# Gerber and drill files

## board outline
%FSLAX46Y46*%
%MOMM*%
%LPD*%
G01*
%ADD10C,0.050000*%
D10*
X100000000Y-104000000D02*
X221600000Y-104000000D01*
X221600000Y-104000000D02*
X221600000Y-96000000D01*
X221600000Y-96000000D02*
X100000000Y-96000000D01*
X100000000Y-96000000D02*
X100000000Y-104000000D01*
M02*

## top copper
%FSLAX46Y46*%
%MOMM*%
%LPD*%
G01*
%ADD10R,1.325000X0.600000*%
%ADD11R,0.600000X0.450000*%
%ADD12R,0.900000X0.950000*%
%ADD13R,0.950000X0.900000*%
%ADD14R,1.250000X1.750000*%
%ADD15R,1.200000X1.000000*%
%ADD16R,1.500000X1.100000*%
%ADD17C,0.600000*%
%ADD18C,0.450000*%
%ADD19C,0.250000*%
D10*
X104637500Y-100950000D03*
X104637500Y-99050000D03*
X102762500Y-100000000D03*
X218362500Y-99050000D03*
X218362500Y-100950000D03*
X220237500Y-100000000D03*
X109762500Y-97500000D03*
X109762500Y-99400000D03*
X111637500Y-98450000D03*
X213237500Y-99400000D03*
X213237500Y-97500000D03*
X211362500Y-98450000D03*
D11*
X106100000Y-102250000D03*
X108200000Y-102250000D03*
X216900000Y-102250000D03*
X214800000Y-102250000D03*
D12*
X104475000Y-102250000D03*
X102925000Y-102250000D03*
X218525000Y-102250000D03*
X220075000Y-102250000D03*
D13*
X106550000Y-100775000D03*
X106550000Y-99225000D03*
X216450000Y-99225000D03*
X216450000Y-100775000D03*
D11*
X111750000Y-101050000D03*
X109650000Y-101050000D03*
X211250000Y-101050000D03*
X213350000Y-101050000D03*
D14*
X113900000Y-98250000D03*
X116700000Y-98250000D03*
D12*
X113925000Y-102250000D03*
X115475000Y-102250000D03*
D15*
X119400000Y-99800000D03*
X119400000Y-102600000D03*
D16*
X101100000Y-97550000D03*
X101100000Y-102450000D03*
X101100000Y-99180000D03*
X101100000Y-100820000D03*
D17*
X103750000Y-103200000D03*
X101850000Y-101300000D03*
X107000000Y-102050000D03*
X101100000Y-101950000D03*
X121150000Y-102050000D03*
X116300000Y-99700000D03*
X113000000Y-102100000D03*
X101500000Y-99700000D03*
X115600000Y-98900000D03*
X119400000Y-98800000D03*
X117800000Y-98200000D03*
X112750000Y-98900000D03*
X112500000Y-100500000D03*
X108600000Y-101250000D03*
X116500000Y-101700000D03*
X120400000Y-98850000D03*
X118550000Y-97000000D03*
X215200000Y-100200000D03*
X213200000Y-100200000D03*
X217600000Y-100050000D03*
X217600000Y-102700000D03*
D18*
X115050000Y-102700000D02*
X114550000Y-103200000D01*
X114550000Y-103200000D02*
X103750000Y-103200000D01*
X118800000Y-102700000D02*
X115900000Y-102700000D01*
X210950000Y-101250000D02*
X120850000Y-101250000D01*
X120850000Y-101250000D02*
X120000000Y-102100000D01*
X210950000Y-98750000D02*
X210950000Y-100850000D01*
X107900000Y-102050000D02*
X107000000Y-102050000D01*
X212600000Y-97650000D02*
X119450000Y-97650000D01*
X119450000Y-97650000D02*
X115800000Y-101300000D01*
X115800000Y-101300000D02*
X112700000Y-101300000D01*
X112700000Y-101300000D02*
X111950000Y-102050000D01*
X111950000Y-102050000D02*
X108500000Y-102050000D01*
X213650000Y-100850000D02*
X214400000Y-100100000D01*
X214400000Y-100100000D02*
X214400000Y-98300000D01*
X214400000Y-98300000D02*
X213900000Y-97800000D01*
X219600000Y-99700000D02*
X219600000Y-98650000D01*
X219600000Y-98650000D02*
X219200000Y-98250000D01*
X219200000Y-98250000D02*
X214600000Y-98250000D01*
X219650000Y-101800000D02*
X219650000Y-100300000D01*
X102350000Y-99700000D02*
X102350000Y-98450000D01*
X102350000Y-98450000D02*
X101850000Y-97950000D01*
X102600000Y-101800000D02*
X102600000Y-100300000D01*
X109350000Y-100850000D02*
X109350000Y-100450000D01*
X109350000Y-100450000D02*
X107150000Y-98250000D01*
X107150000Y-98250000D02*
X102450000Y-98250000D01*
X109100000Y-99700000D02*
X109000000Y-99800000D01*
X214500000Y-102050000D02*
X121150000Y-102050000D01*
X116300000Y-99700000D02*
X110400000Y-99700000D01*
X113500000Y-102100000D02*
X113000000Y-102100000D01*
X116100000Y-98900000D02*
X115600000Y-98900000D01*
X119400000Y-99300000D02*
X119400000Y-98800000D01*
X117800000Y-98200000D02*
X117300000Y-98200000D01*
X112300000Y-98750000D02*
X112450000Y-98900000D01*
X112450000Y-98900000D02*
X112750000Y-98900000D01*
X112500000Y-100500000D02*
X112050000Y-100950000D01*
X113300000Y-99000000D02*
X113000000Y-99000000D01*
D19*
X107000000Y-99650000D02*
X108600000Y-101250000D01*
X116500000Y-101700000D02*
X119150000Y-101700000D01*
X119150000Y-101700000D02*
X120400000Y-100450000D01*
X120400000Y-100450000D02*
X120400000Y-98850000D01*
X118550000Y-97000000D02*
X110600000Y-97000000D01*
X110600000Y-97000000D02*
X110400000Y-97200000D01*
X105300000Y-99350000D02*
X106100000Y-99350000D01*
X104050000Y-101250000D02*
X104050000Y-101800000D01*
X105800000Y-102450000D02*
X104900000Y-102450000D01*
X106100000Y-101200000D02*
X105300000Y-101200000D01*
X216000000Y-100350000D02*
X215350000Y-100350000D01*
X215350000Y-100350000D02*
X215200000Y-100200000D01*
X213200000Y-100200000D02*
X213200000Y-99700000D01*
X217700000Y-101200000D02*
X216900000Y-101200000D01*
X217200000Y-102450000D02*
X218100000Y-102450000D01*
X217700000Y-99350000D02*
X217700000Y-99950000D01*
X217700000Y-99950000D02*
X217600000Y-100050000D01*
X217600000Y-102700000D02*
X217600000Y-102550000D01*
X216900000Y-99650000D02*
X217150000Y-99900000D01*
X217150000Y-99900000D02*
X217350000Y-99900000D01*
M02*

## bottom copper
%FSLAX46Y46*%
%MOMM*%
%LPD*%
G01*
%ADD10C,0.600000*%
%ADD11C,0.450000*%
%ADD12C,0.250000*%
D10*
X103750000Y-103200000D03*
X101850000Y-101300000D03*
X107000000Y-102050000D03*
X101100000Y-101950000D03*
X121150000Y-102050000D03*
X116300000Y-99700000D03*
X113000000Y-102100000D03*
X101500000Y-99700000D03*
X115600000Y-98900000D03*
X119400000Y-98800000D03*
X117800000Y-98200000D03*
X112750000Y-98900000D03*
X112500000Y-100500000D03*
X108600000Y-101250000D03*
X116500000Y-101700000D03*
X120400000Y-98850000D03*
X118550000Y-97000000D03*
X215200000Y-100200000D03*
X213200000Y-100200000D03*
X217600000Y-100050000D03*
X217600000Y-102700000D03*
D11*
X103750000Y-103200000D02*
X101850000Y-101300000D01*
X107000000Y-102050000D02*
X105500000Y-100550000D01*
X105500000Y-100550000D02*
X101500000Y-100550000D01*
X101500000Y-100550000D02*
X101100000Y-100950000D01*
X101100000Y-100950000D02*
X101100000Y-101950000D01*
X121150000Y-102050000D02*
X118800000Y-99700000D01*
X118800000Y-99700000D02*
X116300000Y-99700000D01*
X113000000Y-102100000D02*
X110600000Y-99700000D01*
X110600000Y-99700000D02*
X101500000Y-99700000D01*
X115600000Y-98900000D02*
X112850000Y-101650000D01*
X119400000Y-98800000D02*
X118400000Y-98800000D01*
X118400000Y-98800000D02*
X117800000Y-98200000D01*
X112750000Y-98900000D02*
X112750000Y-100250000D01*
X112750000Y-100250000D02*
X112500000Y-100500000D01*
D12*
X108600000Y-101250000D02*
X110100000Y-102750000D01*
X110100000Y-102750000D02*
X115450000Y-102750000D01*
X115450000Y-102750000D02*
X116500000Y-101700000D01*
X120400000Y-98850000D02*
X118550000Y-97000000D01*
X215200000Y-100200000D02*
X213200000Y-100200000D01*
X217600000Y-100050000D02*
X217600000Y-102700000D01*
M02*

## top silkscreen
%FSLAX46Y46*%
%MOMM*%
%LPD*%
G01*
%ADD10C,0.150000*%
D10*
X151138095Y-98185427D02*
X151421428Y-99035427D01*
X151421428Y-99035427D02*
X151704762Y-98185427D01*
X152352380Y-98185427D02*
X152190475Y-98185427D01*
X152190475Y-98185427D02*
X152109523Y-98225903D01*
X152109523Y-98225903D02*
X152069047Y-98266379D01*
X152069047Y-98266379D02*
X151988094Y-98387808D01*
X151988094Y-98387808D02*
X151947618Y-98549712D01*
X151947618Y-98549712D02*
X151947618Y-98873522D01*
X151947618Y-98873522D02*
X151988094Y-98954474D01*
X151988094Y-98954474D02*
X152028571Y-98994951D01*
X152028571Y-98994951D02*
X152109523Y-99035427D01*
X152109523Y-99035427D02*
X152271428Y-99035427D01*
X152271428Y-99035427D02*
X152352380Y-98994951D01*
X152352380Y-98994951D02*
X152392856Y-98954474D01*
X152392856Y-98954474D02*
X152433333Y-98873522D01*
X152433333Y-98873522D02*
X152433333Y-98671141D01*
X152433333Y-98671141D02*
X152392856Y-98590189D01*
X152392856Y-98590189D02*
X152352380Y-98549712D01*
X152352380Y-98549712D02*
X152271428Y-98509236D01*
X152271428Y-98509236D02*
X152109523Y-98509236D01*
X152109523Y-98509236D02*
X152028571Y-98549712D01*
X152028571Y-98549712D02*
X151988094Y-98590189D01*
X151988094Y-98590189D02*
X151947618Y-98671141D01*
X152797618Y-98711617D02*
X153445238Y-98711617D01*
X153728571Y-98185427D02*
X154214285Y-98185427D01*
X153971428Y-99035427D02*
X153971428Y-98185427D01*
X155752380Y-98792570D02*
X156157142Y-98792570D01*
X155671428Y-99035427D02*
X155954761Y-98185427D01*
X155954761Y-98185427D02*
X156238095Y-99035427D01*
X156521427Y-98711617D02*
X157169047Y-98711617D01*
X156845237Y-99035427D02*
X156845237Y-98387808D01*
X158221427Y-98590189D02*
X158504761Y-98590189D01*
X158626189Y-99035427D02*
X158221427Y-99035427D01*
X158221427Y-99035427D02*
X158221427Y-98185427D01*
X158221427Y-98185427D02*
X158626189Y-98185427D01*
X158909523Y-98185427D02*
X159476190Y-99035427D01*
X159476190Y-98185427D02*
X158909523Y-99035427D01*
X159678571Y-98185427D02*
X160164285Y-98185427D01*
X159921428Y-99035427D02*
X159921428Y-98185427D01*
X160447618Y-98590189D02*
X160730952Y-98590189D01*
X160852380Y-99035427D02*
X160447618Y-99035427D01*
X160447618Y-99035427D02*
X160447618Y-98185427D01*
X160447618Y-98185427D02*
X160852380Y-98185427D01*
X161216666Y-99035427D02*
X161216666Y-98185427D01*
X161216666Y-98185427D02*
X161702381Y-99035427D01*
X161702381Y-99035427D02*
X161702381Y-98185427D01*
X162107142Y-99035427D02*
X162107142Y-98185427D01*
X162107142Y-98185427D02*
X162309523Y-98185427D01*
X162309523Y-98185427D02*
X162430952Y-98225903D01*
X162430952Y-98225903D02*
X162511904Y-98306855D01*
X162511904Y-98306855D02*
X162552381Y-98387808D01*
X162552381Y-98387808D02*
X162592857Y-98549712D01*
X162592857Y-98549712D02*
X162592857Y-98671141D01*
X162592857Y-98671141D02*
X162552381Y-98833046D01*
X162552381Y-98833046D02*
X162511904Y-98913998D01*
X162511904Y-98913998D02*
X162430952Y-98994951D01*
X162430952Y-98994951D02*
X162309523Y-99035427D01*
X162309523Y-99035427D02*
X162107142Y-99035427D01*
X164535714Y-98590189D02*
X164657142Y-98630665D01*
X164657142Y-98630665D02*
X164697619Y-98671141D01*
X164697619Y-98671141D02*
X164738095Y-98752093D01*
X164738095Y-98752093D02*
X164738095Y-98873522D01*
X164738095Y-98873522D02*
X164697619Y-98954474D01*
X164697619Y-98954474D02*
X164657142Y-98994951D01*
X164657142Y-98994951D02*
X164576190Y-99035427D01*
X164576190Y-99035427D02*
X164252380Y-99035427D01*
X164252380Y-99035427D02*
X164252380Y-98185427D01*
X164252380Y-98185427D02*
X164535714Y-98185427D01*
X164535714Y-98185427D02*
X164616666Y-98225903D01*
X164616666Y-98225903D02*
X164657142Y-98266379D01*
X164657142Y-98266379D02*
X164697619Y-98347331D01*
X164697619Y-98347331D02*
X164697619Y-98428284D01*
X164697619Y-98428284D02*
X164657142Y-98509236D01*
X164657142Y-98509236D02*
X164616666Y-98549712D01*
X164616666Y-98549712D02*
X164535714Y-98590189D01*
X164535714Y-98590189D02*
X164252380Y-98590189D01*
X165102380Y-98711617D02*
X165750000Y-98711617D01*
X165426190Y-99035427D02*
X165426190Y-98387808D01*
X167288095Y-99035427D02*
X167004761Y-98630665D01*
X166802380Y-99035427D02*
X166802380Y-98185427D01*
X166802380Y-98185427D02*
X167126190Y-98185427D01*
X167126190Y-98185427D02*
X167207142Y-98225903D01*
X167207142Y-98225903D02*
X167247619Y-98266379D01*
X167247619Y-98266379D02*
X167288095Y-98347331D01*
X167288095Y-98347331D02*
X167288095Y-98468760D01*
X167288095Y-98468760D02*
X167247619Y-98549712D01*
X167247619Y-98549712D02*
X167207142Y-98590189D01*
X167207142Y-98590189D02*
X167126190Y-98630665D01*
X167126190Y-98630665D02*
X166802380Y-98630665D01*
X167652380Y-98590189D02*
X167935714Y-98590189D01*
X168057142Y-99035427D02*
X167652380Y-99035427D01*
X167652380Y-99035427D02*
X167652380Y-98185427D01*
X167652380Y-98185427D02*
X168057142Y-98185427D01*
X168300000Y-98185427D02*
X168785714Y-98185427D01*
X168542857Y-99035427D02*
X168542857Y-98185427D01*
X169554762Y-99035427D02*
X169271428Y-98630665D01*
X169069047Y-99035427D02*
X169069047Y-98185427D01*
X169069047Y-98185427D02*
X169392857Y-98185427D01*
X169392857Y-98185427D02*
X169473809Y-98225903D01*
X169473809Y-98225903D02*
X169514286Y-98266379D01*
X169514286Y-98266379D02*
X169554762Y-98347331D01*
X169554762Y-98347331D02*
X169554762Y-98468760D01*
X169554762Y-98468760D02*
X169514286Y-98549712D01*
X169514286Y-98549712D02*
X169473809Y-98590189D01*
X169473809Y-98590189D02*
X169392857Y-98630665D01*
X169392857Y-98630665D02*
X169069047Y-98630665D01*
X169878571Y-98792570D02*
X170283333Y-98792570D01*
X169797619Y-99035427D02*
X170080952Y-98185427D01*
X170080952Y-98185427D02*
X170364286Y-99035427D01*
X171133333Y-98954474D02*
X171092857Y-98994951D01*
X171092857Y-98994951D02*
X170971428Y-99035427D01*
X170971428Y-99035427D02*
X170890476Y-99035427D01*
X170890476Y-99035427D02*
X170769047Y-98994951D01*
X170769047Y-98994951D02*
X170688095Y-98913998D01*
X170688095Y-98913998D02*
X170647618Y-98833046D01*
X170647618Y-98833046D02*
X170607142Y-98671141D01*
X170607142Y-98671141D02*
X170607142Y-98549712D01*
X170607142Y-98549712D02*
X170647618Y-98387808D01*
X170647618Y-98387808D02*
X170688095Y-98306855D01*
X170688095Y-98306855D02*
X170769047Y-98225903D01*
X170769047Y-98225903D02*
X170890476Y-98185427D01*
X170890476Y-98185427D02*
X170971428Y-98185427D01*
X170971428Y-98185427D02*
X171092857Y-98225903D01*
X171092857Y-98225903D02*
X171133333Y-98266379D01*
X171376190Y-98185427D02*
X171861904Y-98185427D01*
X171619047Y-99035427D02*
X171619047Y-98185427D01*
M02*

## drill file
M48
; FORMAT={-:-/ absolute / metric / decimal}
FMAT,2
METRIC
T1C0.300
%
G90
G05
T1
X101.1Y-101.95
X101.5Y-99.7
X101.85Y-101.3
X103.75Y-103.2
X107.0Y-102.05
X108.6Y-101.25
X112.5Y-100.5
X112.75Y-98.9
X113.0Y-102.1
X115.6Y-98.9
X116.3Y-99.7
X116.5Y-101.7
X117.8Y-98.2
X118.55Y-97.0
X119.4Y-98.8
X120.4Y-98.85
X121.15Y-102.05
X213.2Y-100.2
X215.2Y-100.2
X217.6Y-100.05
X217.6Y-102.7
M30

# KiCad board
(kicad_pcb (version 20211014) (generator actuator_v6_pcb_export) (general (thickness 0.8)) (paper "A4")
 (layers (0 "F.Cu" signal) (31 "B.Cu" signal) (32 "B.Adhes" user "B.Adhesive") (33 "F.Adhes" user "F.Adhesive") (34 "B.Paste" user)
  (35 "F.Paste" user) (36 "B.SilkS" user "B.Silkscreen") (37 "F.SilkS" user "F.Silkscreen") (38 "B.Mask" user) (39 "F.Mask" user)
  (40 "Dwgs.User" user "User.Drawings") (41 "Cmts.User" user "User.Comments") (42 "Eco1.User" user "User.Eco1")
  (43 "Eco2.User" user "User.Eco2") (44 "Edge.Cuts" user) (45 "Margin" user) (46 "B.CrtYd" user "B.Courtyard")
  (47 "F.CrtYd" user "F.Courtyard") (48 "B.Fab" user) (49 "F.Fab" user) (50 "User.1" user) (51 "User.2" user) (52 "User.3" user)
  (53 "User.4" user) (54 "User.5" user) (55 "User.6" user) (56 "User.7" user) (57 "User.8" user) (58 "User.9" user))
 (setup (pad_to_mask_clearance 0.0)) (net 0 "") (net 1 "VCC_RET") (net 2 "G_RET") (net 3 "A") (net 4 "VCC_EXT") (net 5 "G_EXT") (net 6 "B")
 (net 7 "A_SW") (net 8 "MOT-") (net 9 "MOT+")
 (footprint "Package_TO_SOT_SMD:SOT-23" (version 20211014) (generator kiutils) (layer "F.Cu") (at 103.7 100.0 180)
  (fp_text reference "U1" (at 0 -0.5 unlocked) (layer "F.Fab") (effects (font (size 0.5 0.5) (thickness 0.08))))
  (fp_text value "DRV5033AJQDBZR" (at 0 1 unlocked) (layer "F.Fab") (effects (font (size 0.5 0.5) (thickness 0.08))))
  (pad "1" smd rect (at -0.9375 -0.95 180) (size 1.325 0.6) (layers "F.Cu" "F.Mask" "F.Paste") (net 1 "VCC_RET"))
  (pad "2" smd rect (at -0.9375 0.95 180) (size 1.325 0.6) (layers "F.Cu" "F.Mask" "F.Paste") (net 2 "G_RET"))
  (pad "3" smd rect (at 0.9375 0.0 180) (size 1.325 0.6) (layers "F.Cu" "F.Mask" "F.Paste") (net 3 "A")))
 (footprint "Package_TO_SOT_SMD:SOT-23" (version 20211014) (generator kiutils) (layer "F.Cu") (at 219.3 100.0)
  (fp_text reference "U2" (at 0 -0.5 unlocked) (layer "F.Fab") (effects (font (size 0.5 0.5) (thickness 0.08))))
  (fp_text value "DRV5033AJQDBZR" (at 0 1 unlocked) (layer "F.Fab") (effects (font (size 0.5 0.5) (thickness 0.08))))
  (pad "1" smd rect (at -0.9375 -0.95) (size 1.325 0.6) (layers "F.Cu" "F.Mask" "F.Paste") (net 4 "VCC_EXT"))
  (pad "2" smd rect (at -0.9375 0.95) (size 1.325 0.6) (layers "F.Cu" "F.Mask" "F.Paste") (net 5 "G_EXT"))
  (pad "3" smd rect (at 0.9375 0.0) (size 1.325 0.6) (layers "F.Cu" "F.Mask" "F.Paste") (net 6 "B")))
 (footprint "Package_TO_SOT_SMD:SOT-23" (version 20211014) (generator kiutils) (layer "F.Cu") (at 110.7 98.45)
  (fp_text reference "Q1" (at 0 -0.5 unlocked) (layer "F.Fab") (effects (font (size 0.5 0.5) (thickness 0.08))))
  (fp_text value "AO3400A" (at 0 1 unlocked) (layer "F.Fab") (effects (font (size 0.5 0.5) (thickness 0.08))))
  (pad "1" smd rect (at -0.9375 -0.95) (size 1.325 0.6) (layers "F.Cu" "F.Mask" "F.Paste") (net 2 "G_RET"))
  (pad "2" smd rect (at -0.9375 0.95) (size 1.325 0.6) (layers "F.Cu" "F.Mask" "F.Paste") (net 3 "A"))
  (pad "3" smd rect (at 0.9375 0.0) (size 1.325 0.6) (layers "F.Cu" "F.Mask" "F.Paste") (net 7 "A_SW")))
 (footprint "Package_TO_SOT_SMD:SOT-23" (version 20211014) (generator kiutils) (layer "F.Cu") (at 212.3 98.45 180)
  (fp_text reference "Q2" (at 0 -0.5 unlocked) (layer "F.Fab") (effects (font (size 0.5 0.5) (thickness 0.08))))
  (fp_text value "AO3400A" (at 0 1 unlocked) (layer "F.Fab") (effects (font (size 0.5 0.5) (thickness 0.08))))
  (pad "1" smd rect (at -0.9375 -0.95 180) (size 1.325 0.6) (layers "F.Cu" "F.Mask" "F.Paste") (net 5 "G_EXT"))
  (pad "2" smd rect (at -0.9375 0.95 180) (size 1.325 0.6) (layers "F.Cu" "F.Mask" "F.Paste") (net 6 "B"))
  (pad "3" smd rect (at 0.9375 0.0 180) (size 1.325 0.6) (layers "F.Cu" "F.Mask" "F.Paste") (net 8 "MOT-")))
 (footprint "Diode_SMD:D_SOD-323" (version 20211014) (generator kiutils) (layer "F.Cu") (at 107.15 102.25)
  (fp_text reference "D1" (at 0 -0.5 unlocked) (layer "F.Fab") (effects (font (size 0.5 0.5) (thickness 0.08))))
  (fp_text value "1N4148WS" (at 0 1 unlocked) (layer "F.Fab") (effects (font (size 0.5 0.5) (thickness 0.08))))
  (pad "1" smd rect (at -1.05 0.0) (size 0.6 0.45) (layers "F.Cu" "F.Mask" "F.Paste") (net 1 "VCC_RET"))
  (pad "2" smd rect (at 1.05 0.0) (size 0.6 0.45) (layers "F.Cu" "F.Mask" "F.Paste") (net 6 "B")))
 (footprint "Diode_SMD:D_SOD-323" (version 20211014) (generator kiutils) (layer "F.Cu") (at 215.85 102.25 180)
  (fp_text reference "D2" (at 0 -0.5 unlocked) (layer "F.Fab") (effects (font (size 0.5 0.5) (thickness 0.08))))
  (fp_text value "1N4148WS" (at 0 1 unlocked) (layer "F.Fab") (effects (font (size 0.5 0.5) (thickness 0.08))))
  (pad "1" smd rect (at -1.05 0.0 180) (size 0.6 0.45) (layers "F.Cu" "F.Mask" "F.Paste") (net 4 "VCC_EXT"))
  (pad "2" smd rect (at 1.05 0.0 180) (size 0.6 0.45) (layers "F.Cu" "F.Mask" "F.Paste") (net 3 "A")))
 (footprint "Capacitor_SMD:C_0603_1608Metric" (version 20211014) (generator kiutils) (layer "F.Cu") (at 103.7 102.25 180)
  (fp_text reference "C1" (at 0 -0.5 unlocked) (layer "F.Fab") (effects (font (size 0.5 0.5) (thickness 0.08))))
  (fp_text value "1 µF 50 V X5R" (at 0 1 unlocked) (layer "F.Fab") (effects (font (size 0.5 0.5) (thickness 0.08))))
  (pad "1" smd rect (at -0.775 0.0 180) (size 0.9 0.95) (layers "F.Cu" "F.Mask" "F.Paste") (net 1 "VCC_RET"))
  (pad "2" smd rect (at 0.775 0.0 180) (size 0.9 0.95) (layers "F.Cu" "F.Mask" "F.Paste") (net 3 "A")))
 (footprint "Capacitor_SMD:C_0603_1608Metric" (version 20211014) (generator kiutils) (layer "F.Cu") (at 219.3 102.25)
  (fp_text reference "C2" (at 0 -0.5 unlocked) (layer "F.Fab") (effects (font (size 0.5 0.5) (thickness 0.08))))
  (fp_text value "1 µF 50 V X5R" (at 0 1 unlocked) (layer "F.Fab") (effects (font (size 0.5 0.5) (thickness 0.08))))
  (pad "1" smd rect (at -0.775 0.0) (size 0.9 0.95) (layers "F.Cu" "F.Mask" "F.Paste") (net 4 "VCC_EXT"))
  (pad "2" smd rect (at 0.775 0.0) (size 0.9 0.95) (layers "F.Cu" "F.Mask" "F.Paste") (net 6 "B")))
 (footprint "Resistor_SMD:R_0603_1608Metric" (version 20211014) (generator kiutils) (layer "F.Cu") (at 106.55 100.0 90)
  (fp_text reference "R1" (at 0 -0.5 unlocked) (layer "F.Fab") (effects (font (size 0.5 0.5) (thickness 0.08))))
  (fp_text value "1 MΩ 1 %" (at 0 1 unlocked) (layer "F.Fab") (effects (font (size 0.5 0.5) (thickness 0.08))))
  (pad "1" smd rect (at -0.775 0.0 90) (size 0.9 0.95) (layers "F.Cu" "F.Mask" "F.Paste") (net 1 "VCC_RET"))
  (pad "2" smd rect (at 0.775 0.0 90) (size 0.9 0.95) (layers "F.Cu" "F.Mask" "F.Paste") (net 2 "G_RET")))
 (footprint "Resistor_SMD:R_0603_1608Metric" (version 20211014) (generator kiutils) (layer "F.Cu") (at 216.45 100.0 270)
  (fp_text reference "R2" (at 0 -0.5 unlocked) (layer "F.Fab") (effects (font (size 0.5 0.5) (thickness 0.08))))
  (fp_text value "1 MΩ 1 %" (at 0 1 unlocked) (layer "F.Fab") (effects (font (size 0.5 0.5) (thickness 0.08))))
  (pad "1" smd rect (at -0.775 0.0 270) (size 0.9 0.95) (layers "F.Cu" "F.Mask" "F.Paste") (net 4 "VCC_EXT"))
  (pad "2" smd rect (at 0.775 0.0 270) (size 0.9 0.95) (layers "F.Cu" "F.Mask" "F.Paste") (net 5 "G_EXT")))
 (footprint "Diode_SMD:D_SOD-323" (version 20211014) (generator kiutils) (layer "F.Cu") (at 110.7 101.05 180)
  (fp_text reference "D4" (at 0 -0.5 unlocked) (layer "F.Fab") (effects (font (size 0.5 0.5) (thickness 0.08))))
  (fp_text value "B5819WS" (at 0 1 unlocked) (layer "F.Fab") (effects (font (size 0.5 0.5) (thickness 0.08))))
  (pad "1" smd rect (at -1.05 0.0 180) (size 0.6 0.45) (layers "F.Cu" "F.Mask" "F.Paste") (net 7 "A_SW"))
  (pad "2" smd rect (at 1.05 0.0 180) (size 0.6 0.45) (layers "F.Cu" "F.Mask" "F.Paste") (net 3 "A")))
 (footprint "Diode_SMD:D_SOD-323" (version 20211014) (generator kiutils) (layer "F.Cu") (at 212.3 101.05)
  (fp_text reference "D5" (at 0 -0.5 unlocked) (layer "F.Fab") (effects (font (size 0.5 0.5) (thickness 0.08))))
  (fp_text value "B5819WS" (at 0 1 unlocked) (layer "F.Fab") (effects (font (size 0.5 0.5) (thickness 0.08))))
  (pad "1" smd rect (at -1.05 0.0) (size 0.6 0.45) (layers "F.Cu" "F.Mask" "F.Paste") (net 8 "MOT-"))
  (pad "2" smd rect (at 1.05 0.0) (size 0.6 0.45) (layers "F.Cu" "F.Mask" "F.Paste") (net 6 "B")))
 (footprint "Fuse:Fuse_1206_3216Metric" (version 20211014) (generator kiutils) (layer "F.Cu") (at 115.3 98.25)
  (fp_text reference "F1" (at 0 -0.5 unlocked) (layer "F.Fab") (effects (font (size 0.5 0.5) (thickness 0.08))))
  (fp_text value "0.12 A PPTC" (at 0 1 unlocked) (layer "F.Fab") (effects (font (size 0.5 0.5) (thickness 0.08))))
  (pad "1" smd rect (at -1.4 0.0) (size 1.25 1.75) (layers "F.Cu" "F.Mask" "F.Paste") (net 7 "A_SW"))
  (pad "2" smd rect (at 1.4 0.0) (size 1.25 1.75) (layers "F.Cu" "F.Mask" "F.Paste") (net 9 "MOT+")))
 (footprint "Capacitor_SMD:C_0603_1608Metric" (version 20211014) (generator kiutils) (layer "F.Cu") (at 114.7 102.25)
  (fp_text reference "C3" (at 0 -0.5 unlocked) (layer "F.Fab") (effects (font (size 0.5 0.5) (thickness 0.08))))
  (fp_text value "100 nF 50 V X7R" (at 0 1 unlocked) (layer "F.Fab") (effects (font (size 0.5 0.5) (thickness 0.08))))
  (pad "1" smd rect (at -0.775 0.0) (size 0.9 0.95) (layers "F.Cu" "F.Mask" "F.Paste") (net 9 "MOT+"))
  (pad "2" smd rect (at 0.775 0.0) (size 0.9 0.95) (layers "F.Cu" "F.Mask" "F.Paste") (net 8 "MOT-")))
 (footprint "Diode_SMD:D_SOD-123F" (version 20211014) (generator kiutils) (layer "F.Cu") (at 119.4 101.2 270)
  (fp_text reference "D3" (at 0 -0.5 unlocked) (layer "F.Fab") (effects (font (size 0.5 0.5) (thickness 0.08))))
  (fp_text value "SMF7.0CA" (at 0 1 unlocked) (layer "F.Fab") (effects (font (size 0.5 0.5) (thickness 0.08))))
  (pad "1" smd rect (at -1.4 0.0 270) (size 1.0 1.2) (layers "F.Cu" "F.Mask" "F.Paste") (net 9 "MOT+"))
  (pad "2" smd rect (at 1.4 0.0 270) (size 1.0 1.2) (layers "F.Cu" "F.Mask" "F.Paste") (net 8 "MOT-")))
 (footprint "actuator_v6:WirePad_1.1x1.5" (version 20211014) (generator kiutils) (layer "F.Cu") (at 101.1 97.55)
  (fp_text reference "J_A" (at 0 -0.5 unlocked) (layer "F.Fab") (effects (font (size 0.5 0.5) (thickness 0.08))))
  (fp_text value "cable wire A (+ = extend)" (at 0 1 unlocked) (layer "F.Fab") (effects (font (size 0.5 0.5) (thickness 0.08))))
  (pad "1" smd rect (at 0.0 0.0) (size 1.5 1.1) (layers "F.Cu" "F.Mask") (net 3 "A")))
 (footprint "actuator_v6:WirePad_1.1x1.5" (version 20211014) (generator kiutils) (layer "F.Cu") (at 101.1 102.45)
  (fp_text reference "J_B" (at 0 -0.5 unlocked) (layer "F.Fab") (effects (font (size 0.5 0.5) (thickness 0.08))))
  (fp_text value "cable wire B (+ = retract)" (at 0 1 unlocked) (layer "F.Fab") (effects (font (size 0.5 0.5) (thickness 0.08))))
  (pad "1" smd rect (at 0.0 0.0) (size 1.5 1.1) (layers "F.Cu" "F.Mask") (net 6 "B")))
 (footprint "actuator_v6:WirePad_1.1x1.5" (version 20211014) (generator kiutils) (layer "F.Cu") (at 101.1 99.18)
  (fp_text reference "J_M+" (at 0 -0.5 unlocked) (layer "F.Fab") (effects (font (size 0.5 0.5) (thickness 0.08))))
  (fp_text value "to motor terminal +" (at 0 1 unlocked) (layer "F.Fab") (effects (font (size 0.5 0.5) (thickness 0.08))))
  (pad "1" smd rect (at 0.0 0.0) (size 1.5 1.1) (layers "F.Cu" "F.Mask") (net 9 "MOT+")))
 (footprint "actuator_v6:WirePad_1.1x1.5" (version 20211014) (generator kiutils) (layer "F.Cu") (at 101.1 100.82)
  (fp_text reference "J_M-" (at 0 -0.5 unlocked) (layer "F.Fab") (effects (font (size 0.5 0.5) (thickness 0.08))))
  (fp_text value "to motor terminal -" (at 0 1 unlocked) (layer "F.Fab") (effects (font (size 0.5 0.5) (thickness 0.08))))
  (pad "1" smd rect (at 0.0 0.0) (size 1.5 1.1) (layers "F.Cu" "F.Mask") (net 8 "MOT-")))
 (gr_line (start 100.0 104.0) (end 221.6 104.0) (layer "Edge.Cuts") (width 0.05))
 (gr_line (start 221.6 104.0) (end 221.6 96.0) (layer "Edge.Cuts") (width 0.05))
 (gr_line (start 221.6 96.0) (end 100.0 96.0) (layer "Edge.Cuts") (width 0.05))
 (gr_line (start 100.0 96.0) (end 100.0 104.0) (layer "Edge.Cuts") (width 0.05))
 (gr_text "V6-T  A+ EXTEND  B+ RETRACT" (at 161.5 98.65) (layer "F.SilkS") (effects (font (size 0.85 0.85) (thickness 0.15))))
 (segment (start 115.05 102.7) (end 114.55 103.2) (width 0.45) (layer "F.Cu") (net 8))
 (segment (start 114.55 103.2) (end 103.75 103.2) (width 0.45) (layer "F.Cu") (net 8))
 (segment (start 103.75 103.2) (end 101.85 101.3) (width 0.45) (layer "B.Cu") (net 8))
 (segment (start 118.8 102.7) (end 115.9 102.7) (width 0.45) (layer "F.Cu") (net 8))
 (segment (start 210.95 101.25) (end 120.85 101.25) (width 0.45) (layer "F.Cu") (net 8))
 (segment (start 120.85 101.25) (end 120.0 102.1) (width 0.45) (layer "F.Cu") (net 8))
 (segment (start 210.95 98.75) (end 210.95 100.85) (width 0.45) (layer "F.Cu") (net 8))
 (segment (start 107.9 102.05) (end 107.0 102.05) (width 0.45) (layer "F.Cu") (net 6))
 (segment (start 107.0 102.05) (end 105.5 100.55) (width 0.45) (layer "B.Cu") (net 6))
 (segment (start 105.5 100.55) (end 101.5 100.55) (width 0.45) (layer "B.Cu") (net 6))
 (segment (start 101.5 100.55) (end 101.1 100.95) (width 0.45) (layer "B.Cu") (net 6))
 (segment (start 101.1 100.95) (end 101.1 101.95) (width 0.45) (layer "B.Cu") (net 6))
 (segment (start 212.6 97.65) (end 119.45 97.65) (width 0.45) (layer "F.Cu") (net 6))
 (segment (start 119.45 97.65) (end 115.8 101.3) (width 0.45) (layer "F.Cu") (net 6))
 (segment (start 115.8 101.3) (end 112.7 101.3) (width 0.45) (layer "F.Cu") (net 6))
 (segment (start 112.7 101.3) (end 111.95 102.05) (width 0.45) (layer "F.Cu") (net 6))
 (segment (start 111.95 102.05) (end 108.5 102.05) (width 0.45) (layer "F.Cu") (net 6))
 (segment (start 213.65 100.85) (end 214.4 100.1) (width 0.45) (layer "F.Cu") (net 6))
 (segment (start 214.4 100.1) (end 214.4 98.3) (width 0.45) (layer "F.Cu") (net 6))
 (segment (start 214.4 98.3) (end 213.9 97.8) (width 0.45) (layer "F.Cu") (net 6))
 (segment (start 219.6 99.7) (end 219.6 98.65) (width 0.45) (layer "F.Cu") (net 6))
 (segment (start 219.6 98.65) (end 219.2 98.25) (width 0.45) (layer "F.Cu") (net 6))
 (segment (start 219.2 98.25) (end 214.6 98.25) (width 0.45) (layer "F.Cu") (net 6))
 (segment (start 219.65 101.8) (end 219.65 100.3) (width 0.45) (layer "F.Cu") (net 6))
 (segment (start 102.35 99.7) (end 102.35 98.45) (width 0.45) (layer "F.Cu") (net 3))
 (segment (start 102.35 98.45) (end 101.85 97.95) (width 0.45) (layer "F.Cu") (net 3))
 (segment (start 102.6 101.8) (end 102.6 100.3) (width 0.45) (layer "F.Cu") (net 3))
 (segment (start 109.35 100.85) (end 109.35 100.45) (width 0.45) (layer "F.Cu") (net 3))
 (segment (start 109.35 100.45) (end 107.15 98.25) (width 0.45) (layer "F.Cu") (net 3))
 (segment (start 107.15 98.25) (end 102.45 98.25) (width 0.45) (layer "F.Cu") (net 3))
 (segment (start 109.1 99.7) (end 109.0 99.8) (width 0.45) (layer "F.Cu") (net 3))
 (segment (start 214.5 102.05) (end 121.15 102.05) (width 0.45) (layer "F.Cu") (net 3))
 (segment (start 121.15 102.05) (end 118.8 99.7) (width 0.45) (layer "B.Cu") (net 3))
 (segment (start 118.8 99.7) (end 116.3 99.7) (width 0.45) (layer "B.Cu") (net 3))
 (segment (start 116.3 99.7) (end 110.4 99.7) (width 0.45) (layer "F.Cu") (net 3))
 (segment (start 113.5 102.1) (end 113.0 102.1) (width 0.45) (layer "F.Cu") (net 9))
 (segment (start 113.0 102.1) (end 110.6 99.7) (width 0.45) (layer "B.Cu") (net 9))
 (segment (start 110.6 99.7) (end 101.5 99.7) (width 0.45) (layer "B.Cu") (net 9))
 (segment (start 116.1 98.9) (end 115.6 98.9) (width 0.45) (layer "F.Cu") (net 9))
 (segment (start 115.6 98.9) (end 112.85 101.65) (width 0.45) (layer "B.Cu") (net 9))
 (segment (start 119.4 99.3) (end 119.4 98.8) (width 0.45) (layer "F.Cu") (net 9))
 (segment (start 119.4 98.8) (end 118.4 98.8) (width 0.45) (layer "B.Cu") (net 9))
 (segment (start 118.4 98.8) (end 117.8 98.2) (width 0.45) (layer "B.Cu") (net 9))
 (segment (start 117.8 98.2) (end 117.3 98.2) (width 0.45) (layer "F.Cu") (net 9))
 (segment (start 112.3 98.75) (end 112.45 98.9) (width 0.45) (layer "F.Cu") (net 7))
 (segment (start 112.45 98.9) (end 112.75 98.9) (width 0.45) (layer "F.Cu") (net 7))
 (segment (start 112.75 98.9) (end 112.75 100.25) (width 0.45) (layer "B.Cu") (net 7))
 (segment (start 112.75 100.25) (end 112.5 100.5) (width 0.45) (layer "B.Cu") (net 7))
 (segment (start 112.5 100.5) (end 112.05 100.95) (width 0.45) (layer "F.Cu") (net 7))
 (segment (start 113.3 99.0) (end 113.0 99.0) (width 0.45) (layer "F.Cu") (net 7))
 (segment (start 107.0 99.65) (end 108.6 101.25) (width 0.25) (layer "F.Cu") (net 2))
 (segment (start 108.6 101.25) (end 110.1 102.75) (width 0.25) (layer "B.Cu") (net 2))
 (segment (start 110.1 102.75) (end 115.45 102.75) (width 0.25) (layer "B.Cu") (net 2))
 (segment (start 115.45 102.75) (end 116.5 101.7) (width 0.25) (layer "B.Cu") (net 2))
 (segment (start 116.5 101.7) (end 119.15 101.7) (width 0.25) (layer "F.Cu") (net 2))
 (segment (start 119.15 101.7) (end 120.4 100.45) (width 0.25) (layer "F.Cu") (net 2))
 (segment (start 120.4 100.45) (end 120.4 98.85) (width 0.25) (layer "F.Cu") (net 2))
 (segment (start 120.4 98.85) (end 118.55 97.0) (width 0.25) (layer "B.Cu") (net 2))
 (segment (start 118.55 97.0) (end 110.6 97.0) (width 0.25) (layer "F.Cu") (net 2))
 (segment (start 110.6 97.0) (end 110.4 97.2) (width 0.25) (layer "F.Cu") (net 2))
 (segment (start 105.3 99.35) (end 106.1 99.35) (width 0.25) (layer "F.Cu") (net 2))
 (segment (start 104.05 101.25) (end 104.05 101.8) (width 0.25) (layer "F.Cu") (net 1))
 (segment (start 105.8 102.45) (end 104.9 102.45) (width 0.25) (layer "F.Cu") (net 1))
 (segment (start 106.1 101.2) (end 105.3 101.2) (width 0.25) (layer "F.Cu") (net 1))
 (segment (start 216.0 100.35) (end 215.35 100.35) (width 0.25) (layer "F.Cu") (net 5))
 (segment (start 215.35 100.35) (end 215.2 100.2) (width 0.25) (layer "F.Cu") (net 5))
 (segment (start 215.2 100.2) (end 213.2 100.2) (width 0.25) (layer "B.Cu") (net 5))
 (segment (start 213.2 100.2) (end 213.2 99.7) (width 0.25) (layer "F.Cu") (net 5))
 (segment (start 217.7 101.2) (end 216.9 101.2) (width 0.25) (layer "F.Cu") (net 5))
 (segment (start 217.2 102.45) (end 218.1 102.45) (width 0.25) (layer "F.Cu") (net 4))
 (segment (start 217.7 99.35) (end 217.7 99.95) (width 0.25) (layer "F.Cu") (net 4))
 (segment (start 217.7 99.95) (end 217.6 100.05) (width 0.25) (layer "F.Cu") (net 4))
 (segment (start 217.6 100.05) (end 217.6 102.7) (width 0.25) (layer "B.Cu") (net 4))
 (segment (start 217.6 102.7) (end 217.6 102.55) (width 0.25) (layer "F.Cu") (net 4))
 (segment (start 216.9 99.65) (end 217.15 99.9) (width 0.25) (layer "F.Cu") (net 4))
 (segment (start 217.15 99.9) (end 217.35 99.9) (width 0.25) (layer "F.Cu") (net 4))
 (via (at 103.75 103.2) (size 0.6) (drill 0.3) (layers "F.Cu" "B.Cu") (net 8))
 (via (at 101.85 101.3) (size 0.6) (drill 0.3) (layers "F.Cu" "B.Cu") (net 8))
 (via (at 107.0 102.05) (size 0.6) (drill 0.3) (layers "F.Cu" "B.Cu") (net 6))
 (via (at 101.1 101.95) (size 0.6) (drill 0.3) (layers "F.Cu" "B.Cu") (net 6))
 (via (at 121.15 102.05) (size 0.6) (drill 0.3) (layers "F.Cu" "B.Cu") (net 3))
 (via (at 116.3 99.7) (size 0.6) (drill 0.3) (layers "F.Cu" "B.Cu") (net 3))
 (via (at 113.0 102.1) (size 0.6) (drill 0.3) (layers "F.Cu" "B.Cu") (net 9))
 (via (at 101.5 99.7) (size 0.6) (drill 0.3) (layers "F.Cu" "B.Cu") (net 9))
 (via (at 115.6 98.9) (size 0.6) (drill 0.3) (layers "F.Cu" "B.Cu") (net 9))
 (via (at 119.4 98.8) (size 0.6) (drill 0.3) (layers "F.Cu" "B.Cu") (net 9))
 (via (at 117.8 98.2) (size 0.6) (drill 0.3) (layers "F.Cu" "B.Cu") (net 9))
 (via (at 112.75 98.9) (size 0.6) (drill 0.3) (layers "F.Cu" "B.Cu") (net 7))
 (via (at 112.5 100.5) (size 0.6) (drill 0.3) (layers "F.Cu" "B.Cu") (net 7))
 (via (at 108.6 101.25) (size 0.6) (drill 0.3) (layers "F.Cu" "B.Cu") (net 2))
 (via (at 116.5 101.7) (size 0.6) (drill 0.3) (layers "F.Cu" "B.Cu") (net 2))
 (via (at 120.4 98.85) (size 0.6) (drill 0.3) (layers "F.Cu" "B.Cu") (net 2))
 (via (at 118.55 97.0) (size 0.6) (drill 0.3) (layers "F.Cu" "B.Cu") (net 2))
 (via (at 215.2 100.2) (size 0.6) (drill 0.3) (layers "F.Cu" "B.Cu") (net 5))
 (via (at 213.2 100.2) (size 0.6) (drill 0.3) (layers "F.Cu" "B.Cu") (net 5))
 (via (at 217.6 100.05) (size 0.6) (drill 0.3) (layers "F.Cu" "B.Cu") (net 4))
 (via (at 217.6 102.7) (size 0.6) (drill 0.3) (layers "F.Cu" "B.Cu") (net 4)))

